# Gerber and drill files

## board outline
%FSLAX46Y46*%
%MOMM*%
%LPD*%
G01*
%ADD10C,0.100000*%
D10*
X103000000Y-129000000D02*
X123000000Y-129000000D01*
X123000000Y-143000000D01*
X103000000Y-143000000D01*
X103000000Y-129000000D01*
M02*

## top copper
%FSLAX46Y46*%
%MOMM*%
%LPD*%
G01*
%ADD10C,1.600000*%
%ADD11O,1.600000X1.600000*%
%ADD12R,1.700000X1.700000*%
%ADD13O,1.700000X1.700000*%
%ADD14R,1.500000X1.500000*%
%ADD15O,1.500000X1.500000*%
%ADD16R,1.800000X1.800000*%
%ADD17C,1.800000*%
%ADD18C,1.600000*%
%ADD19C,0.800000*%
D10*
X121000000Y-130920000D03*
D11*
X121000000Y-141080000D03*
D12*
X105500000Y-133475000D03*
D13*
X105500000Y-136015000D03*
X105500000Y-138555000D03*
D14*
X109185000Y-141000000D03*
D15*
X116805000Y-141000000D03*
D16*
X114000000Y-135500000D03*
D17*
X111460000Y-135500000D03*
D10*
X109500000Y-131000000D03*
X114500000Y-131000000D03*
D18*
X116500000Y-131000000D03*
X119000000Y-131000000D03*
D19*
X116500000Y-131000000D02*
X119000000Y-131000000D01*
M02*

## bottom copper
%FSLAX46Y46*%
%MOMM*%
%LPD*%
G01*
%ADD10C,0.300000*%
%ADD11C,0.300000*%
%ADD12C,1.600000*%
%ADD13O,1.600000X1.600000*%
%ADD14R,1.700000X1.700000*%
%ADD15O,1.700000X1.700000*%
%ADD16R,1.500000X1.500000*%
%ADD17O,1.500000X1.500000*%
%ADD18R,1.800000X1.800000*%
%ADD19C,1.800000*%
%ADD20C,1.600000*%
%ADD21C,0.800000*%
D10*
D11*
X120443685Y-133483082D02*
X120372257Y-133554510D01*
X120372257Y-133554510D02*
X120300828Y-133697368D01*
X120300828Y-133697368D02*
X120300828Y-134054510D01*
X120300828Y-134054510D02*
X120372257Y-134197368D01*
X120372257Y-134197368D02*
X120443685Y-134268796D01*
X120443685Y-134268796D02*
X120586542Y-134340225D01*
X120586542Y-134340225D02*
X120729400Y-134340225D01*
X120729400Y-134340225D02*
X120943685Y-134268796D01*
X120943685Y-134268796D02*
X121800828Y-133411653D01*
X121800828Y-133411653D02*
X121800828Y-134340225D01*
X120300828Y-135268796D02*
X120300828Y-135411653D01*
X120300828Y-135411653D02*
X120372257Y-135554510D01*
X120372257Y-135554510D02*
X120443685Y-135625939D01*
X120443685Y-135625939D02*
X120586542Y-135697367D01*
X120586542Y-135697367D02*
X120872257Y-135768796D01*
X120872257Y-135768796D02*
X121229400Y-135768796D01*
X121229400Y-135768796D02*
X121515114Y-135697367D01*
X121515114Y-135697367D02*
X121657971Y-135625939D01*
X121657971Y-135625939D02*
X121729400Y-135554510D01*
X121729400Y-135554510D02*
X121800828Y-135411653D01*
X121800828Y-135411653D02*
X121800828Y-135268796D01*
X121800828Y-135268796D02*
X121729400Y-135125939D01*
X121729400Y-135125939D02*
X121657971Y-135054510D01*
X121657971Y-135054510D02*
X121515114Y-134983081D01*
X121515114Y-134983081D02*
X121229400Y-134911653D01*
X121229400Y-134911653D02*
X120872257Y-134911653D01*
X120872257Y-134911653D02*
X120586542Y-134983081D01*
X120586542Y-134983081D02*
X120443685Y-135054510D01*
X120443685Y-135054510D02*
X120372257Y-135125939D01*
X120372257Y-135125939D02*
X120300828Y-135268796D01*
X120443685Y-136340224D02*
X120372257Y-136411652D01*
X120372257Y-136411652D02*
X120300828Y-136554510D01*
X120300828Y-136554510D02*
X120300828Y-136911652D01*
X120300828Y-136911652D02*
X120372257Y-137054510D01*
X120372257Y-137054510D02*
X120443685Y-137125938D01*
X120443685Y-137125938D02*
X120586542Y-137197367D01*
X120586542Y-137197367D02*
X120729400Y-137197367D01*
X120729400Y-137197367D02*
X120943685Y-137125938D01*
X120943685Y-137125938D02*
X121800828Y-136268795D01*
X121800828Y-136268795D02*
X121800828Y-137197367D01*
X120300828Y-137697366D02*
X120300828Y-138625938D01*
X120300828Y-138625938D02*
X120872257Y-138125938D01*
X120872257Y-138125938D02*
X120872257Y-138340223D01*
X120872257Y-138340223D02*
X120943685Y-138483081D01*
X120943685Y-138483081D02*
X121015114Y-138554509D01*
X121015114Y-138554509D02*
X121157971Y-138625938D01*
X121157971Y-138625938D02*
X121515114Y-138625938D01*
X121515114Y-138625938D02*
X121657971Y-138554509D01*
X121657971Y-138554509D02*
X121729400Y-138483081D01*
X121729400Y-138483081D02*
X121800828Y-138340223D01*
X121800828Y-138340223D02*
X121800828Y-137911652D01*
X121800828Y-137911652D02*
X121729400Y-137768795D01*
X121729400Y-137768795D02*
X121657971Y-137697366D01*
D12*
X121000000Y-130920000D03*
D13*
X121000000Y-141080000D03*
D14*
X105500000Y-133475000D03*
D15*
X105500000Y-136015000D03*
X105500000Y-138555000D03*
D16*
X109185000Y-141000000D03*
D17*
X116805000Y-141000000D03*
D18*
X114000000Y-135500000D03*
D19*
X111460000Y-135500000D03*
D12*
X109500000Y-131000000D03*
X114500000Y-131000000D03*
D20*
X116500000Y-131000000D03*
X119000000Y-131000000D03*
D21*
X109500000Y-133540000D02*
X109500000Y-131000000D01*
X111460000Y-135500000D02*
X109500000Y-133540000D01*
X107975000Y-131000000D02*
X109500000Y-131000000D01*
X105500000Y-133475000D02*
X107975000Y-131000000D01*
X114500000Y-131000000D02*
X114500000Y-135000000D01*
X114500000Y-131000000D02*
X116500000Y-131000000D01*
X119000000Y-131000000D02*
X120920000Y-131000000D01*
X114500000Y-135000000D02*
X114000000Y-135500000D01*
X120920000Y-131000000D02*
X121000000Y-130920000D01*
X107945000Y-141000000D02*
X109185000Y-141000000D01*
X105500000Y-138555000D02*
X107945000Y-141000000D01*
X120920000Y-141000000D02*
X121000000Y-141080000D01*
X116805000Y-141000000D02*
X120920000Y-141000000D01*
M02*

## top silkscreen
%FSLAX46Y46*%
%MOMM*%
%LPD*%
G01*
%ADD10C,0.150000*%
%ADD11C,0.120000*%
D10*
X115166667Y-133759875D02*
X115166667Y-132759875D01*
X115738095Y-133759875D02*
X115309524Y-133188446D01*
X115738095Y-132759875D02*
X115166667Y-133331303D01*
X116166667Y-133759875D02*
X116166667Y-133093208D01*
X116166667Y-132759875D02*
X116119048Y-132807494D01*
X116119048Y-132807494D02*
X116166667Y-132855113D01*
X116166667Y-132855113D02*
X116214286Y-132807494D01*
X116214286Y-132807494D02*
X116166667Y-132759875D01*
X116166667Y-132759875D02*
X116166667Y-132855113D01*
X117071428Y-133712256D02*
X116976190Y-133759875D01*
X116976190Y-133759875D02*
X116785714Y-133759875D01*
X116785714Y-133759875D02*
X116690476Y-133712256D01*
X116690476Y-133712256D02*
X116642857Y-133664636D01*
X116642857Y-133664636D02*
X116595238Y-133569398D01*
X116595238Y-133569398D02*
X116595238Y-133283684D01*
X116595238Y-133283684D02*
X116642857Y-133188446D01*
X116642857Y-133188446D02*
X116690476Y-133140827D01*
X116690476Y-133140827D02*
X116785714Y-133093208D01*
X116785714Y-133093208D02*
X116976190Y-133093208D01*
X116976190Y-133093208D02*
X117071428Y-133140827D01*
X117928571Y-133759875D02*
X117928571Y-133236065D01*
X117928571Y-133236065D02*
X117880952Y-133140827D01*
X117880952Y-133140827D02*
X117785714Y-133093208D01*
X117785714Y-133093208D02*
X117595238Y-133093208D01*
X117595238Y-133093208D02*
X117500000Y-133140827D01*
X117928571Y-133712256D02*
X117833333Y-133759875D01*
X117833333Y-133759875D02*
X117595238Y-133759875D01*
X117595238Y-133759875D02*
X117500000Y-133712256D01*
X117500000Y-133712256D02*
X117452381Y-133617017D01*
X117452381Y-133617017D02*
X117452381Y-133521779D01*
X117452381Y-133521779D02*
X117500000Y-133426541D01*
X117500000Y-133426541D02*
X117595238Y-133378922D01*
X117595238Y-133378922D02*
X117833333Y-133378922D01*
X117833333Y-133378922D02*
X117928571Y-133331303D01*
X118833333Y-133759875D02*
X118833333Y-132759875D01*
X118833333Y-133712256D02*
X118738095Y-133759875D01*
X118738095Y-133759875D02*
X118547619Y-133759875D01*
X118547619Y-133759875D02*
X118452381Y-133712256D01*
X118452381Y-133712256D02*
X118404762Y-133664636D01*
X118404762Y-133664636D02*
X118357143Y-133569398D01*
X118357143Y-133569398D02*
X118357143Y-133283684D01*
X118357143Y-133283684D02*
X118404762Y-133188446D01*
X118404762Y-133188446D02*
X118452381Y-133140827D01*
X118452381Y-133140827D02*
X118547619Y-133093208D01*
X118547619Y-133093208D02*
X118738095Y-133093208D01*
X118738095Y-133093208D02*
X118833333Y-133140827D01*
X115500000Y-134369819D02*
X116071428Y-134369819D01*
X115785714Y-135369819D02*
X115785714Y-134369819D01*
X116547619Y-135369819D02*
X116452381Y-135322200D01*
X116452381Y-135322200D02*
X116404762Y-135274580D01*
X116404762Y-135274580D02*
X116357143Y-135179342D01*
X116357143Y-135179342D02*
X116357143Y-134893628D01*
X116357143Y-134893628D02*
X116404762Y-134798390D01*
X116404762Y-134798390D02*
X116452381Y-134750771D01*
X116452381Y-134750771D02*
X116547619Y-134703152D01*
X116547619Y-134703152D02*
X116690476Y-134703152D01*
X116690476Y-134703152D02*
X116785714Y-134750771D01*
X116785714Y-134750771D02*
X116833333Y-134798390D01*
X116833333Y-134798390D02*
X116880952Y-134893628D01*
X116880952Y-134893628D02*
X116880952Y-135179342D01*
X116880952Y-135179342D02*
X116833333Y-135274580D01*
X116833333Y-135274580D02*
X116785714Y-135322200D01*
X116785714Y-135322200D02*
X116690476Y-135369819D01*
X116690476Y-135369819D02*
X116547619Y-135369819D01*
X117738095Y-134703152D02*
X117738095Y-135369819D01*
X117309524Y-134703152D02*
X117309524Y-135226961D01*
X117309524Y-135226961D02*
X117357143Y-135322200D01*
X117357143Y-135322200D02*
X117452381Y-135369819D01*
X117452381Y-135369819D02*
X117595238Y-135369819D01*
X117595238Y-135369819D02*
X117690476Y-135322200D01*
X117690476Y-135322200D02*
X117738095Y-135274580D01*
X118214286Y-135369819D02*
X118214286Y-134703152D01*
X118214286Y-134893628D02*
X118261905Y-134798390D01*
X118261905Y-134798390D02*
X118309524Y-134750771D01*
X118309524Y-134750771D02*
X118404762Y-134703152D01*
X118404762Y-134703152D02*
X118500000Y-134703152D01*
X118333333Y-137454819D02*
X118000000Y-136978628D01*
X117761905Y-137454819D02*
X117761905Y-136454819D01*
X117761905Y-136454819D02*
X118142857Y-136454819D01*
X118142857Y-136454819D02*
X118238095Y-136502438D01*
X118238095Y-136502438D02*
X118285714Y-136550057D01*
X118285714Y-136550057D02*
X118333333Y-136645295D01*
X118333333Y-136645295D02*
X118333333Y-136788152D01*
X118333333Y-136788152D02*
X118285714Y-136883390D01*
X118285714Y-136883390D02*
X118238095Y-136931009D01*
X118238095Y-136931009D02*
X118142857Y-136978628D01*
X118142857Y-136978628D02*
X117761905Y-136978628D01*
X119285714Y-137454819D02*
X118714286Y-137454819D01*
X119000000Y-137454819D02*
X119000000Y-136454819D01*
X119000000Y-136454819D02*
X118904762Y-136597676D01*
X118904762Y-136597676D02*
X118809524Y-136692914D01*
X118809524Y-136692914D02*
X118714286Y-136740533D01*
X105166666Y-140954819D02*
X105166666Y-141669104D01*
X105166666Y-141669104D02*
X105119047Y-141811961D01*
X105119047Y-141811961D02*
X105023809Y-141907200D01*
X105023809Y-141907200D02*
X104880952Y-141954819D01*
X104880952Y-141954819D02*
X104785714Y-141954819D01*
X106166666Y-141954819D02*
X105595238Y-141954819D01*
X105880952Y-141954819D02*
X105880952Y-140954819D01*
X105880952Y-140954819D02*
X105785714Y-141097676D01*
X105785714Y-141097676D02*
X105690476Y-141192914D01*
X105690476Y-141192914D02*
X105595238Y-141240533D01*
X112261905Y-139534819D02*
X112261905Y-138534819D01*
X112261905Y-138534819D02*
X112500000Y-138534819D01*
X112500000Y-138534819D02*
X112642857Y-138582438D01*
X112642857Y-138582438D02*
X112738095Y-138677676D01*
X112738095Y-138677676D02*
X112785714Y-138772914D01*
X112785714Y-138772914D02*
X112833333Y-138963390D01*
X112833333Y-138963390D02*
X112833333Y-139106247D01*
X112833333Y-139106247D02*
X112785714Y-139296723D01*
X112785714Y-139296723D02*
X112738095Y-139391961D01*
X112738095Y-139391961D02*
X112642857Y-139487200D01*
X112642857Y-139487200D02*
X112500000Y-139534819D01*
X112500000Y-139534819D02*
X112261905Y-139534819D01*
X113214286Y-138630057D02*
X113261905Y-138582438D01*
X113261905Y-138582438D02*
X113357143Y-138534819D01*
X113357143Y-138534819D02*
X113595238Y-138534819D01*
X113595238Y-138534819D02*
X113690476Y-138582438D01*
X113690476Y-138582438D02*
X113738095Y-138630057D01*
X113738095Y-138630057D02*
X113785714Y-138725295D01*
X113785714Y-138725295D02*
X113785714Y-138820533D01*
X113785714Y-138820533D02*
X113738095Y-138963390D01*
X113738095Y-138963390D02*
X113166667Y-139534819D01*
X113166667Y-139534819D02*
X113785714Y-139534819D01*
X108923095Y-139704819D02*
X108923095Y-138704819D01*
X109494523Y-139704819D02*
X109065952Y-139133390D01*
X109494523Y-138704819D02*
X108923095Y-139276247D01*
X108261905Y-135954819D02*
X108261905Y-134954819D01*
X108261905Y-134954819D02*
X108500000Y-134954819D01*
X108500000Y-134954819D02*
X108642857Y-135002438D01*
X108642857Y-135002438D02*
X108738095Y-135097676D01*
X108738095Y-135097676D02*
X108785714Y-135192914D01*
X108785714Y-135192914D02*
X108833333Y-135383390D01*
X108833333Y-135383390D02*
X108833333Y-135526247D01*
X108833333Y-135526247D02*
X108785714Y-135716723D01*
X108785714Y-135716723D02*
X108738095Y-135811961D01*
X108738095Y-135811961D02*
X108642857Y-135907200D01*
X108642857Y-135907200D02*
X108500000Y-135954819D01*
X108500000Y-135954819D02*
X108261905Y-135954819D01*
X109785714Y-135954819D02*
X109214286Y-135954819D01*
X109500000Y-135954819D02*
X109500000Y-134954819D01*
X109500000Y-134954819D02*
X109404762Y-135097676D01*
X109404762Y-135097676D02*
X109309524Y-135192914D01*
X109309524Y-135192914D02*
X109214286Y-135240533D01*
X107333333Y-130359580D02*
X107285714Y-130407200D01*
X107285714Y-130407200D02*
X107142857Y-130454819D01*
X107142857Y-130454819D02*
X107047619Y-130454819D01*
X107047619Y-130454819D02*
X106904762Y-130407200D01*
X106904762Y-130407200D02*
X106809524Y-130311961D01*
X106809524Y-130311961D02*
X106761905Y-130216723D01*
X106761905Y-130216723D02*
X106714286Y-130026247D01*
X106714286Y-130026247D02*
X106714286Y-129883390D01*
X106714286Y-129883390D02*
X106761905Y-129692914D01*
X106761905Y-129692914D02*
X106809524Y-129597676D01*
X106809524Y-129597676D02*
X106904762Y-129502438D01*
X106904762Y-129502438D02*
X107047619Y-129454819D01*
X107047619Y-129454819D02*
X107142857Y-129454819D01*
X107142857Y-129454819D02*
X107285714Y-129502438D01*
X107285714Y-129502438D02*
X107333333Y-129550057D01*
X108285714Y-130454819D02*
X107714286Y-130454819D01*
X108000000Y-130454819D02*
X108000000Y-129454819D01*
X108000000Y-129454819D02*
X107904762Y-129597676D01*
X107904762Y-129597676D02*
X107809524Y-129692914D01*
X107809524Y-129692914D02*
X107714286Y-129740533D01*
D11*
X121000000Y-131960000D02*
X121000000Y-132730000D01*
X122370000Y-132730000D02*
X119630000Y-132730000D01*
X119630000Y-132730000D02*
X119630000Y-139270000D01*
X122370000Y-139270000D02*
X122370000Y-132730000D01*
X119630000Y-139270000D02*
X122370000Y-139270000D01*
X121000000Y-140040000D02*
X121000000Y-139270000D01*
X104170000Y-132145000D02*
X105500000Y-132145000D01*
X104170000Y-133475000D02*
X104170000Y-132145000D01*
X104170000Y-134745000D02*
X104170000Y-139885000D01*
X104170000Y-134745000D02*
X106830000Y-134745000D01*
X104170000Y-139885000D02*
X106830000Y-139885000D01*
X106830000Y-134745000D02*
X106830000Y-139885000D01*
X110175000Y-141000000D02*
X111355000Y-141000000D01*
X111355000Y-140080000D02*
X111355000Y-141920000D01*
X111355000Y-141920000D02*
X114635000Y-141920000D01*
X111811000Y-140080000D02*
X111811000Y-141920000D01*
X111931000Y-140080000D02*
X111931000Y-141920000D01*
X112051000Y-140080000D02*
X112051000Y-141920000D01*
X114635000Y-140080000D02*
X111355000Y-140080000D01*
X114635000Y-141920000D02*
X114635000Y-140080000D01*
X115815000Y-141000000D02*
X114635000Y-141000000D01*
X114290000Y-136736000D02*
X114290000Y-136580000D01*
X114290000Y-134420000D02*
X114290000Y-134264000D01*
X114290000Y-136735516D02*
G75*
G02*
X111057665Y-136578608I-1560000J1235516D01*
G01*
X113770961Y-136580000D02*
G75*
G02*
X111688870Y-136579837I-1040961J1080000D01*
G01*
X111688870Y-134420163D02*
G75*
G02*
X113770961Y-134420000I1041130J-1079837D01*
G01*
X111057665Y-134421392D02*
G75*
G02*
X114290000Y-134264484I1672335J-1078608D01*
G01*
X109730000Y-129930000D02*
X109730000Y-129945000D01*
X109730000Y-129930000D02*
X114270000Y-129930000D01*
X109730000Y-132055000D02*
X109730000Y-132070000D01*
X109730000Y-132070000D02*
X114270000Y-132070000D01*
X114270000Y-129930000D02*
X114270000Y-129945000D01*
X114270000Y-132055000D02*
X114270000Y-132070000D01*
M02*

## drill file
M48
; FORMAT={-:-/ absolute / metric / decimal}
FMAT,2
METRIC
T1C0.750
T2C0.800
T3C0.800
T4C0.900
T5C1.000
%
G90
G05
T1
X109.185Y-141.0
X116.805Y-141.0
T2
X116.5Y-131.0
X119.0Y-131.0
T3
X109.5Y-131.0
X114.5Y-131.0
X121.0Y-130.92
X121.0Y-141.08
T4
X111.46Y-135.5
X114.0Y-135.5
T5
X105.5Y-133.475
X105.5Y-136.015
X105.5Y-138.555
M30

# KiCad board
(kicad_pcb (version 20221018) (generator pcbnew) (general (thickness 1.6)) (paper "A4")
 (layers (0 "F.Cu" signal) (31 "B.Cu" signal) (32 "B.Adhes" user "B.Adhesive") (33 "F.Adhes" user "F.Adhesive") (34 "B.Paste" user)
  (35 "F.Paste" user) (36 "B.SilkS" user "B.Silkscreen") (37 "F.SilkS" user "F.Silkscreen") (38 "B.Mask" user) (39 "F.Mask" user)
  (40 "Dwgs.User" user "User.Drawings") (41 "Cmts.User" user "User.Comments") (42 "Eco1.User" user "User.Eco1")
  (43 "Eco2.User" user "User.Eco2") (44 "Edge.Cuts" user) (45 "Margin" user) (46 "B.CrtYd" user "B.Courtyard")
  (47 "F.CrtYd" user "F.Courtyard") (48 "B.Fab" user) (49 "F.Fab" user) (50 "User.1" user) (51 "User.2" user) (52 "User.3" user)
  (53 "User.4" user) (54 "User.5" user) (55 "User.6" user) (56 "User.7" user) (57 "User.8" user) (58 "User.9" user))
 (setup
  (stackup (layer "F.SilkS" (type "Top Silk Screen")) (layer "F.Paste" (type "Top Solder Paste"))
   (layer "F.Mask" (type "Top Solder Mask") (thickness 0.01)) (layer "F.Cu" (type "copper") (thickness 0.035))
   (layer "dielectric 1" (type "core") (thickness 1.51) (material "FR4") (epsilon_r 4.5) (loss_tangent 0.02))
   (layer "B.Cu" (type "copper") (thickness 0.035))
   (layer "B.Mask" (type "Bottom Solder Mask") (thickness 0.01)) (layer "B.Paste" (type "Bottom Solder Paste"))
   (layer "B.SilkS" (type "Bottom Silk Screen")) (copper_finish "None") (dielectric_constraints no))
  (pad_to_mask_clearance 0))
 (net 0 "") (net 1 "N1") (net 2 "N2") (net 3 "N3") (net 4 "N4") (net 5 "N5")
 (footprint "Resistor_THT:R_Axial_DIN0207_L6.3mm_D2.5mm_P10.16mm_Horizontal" (layer "F.Cu") (at 121 130.92 -90)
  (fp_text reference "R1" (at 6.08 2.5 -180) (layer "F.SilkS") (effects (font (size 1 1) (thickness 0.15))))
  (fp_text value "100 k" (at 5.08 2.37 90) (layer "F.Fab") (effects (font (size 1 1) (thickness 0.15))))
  (fp_line (start 1.04 0) (end 1.81 0) (stroke (width 0.12) (type solid)) (layer "F.SilkS"))
  (fp_line (start 1.81 -1.37) (end 1.81 1.37) (stroke (width 0.12) (type solid)) (layer "F.SilkS"))
  (fp_line (start 1.81 1.37) (end 8.35 1.37) (stroke (width 0.12) (type solid)) (layer "F.SilkS"))
  (fp_line (start 8.35 -1.37) (end 1.81 -1.37) (stroke (width 0.12) (type solid)) (layer "F.SilkS"))
  (fp_line (start 8.35 1.37) (end 8.35 -1.37) (stroke (width 0.12) (type solid)) (layer "F.SilkS"))
  (fp_line (start 9.12 0) (end 8.35 0) (stroke (width 0.12) (type solid)) (layer "F.SilkS"))
  (pad "1" thru_hole circle (at 0 0 270) (size 1.6 1.6) (drill 0.8) (layers "*.Cu" "*.Mask") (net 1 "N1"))
  (pad "2" thru_hole oval (at 10.16 0 270) (size 1.6 1.6) (drill 0.8) (layers "*.Cu" "*.Mask") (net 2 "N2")))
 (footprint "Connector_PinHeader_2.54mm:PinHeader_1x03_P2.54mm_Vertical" (layer "F.Cu") (at 105.5 133.475)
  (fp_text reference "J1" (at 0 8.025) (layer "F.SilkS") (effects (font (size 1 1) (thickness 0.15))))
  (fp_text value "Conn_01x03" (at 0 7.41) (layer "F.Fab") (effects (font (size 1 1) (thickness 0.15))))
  (fp_line (start -1.33 -1.33) (end 0 -1.33) (stroke (width 0.12) (type solid)) (layer "F.SilkS"))
  (fp_line (start -1.33 0) (end -1.33 -1.33) (stroke (width 0.12) (type solid)) (layer "F.SilkS"))
  (fp_line (start -1.33 1.27) (end -1.33 6.41) (stroke (width 0.12) (type solid)) (layer "F.SilkS"))
  (fp_line (start -1.33 1.27) (end 1.33 1.27) (stroke (width 0.12) (type solid)) (layer "F.SilkS"))
  (fp_line (start -1.33 6.41) (end 1.33 6.41) (stroke (width 0.12) (type solid)) (layer "F.SilkS"))
  (fp_line (start 1.33 1.27) (end 1.33 6.41) (stroke (width 0.12) (type solid)) (layer "F.SilkS"))
  (pad "1" thru_hole rect (at 0 0) (size 1.7 1.7) (drill 1) (layers "*.Cu" "*.Mask") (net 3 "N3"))
  (pad "2" thru_hole oval (at 0 2.54) (size 1.7 1.7) (drill 1) (layers "*.Cu" "*.Mask") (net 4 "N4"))
  (pad "3" thru_hole oval (at 0 5.08) (size 1.7 1.7) (drill 1) (layers "*.Cu" "*.Mask") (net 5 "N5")))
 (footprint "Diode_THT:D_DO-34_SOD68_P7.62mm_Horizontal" (layer "F.Cu") (at 109.185 141)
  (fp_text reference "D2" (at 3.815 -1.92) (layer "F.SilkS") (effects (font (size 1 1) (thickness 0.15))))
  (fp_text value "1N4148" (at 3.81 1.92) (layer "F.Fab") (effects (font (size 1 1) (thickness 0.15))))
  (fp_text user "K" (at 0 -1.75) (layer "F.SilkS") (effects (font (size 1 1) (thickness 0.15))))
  (fp_line (start 0.99 0) (end 2.17 0) (stroke (width 0.12) (type solid)) (layer "F.SilkS"))
  (fp_line (start 2.17 -0.92) (end 2.17 0.92) (stroke (width 0.12) (type solid)) (layer "F.SilkS"))
  (fp_line (start 2.17 0.92) (end 5.45 0.92) (stroke (width 0.12) (type solid)) (layer "F.SilkS"))
  (fp_line (start 2.626 -0.92) (end 2.626 0.92) (stroke (width 0.12) (type solid)) (layer "F.SilkS"))
  (fp_line (start 2.746 -0.92) (end 2.746 0.92) (stroke (width 0.12) (type solid)) (layer "F.SilkS"))
  (fp_line (start 2.866 -0.92) (end 2.866 0.92) (stroke (width 0.12) (type solid)) (layer "F.SilkS"))
  (fp_line (start 5.45 -0.92) (end 2.17 -0.92) (stroke (width 0.12) (type solid)) (layer "F.SilkS"))
  (fp_line (start 5.45 0.92) (end 5.45 -0.92) (stroke (width 0.12) (type solid)) (layer "F.SilkS"))
  (fp_line (start 6.63 0) (end 5.45 0) (stroke (width 0.12) (type solid)) (layer "F.SilkS"))
  (pad "1" thru_hole rect (at 0 0) (size 1.5 1.5) (drill 0.75) (layers "*.Cu" "*.Mask") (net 5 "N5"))
  (pad "2" thru_hole oval (at 7.62 0) (size 1.5 1.5) (drill 0.75) (layers "*.Cu" "*.Mask") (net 2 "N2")))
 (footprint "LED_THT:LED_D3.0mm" (layer "F.Cu") (at 114 135.5 180)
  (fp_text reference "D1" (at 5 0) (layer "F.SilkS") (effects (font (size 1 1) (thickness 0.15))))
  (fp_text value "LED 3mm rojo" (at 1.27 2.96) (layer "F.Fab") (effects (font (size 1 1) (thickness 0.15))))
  (fp_line (start -0.29 -1.236) (end -0.29 -1.08) (stroke (width 0.12) (type solid)) (layer "F.SilkS"))
  (fp_line (start -0.29 1.08) (end -0.29 1.236) (stroke (width 0.12) (type solid)) (layer "F.SilkS"))
  (fp_arc (start -0.29 -1.235516) (mid 1.366487 -1.987659) (end 2.942335 -1.078608) (stroke (width 0.12) (type solid)) (layer "F.SilkS"))
  (fp_arc (start 0.229039 -1.08) (mid 1.270117 -1.5) (end 2.31113 -1.079837) (stroke (width 0.12) (type solid)) (layer "F.SilkS"))
  (fp_arc (start 2.31113 1.079837) (mid 1.270117 1.5) (end 0.229039 1.08) (stroke (width 0.12) (type solid)) (layer "F.SilkS"))
  (fp_arc (start 2.942335 1.078608) (mid 1.366487 1.987659) (end -0.29 1.235516) (stroke (width 0.12) (type solid)) (layer "F.SilkS"))
  (pad "1" thru_hole rect (at 0 0 180) (size 1.8 1.8) (drill 0.9) (layers "*.Cu" "*.Mask") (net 1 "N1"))
  (pad "2" thru_hole circle (at 2.54 0 180) (size 1.8 1.8) (drill 0.9) (layers "*.Cu" "*.Mask") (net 3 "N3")))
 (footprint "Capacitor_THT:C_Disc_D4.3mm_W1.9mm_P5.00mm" (layer "F.Cu") (at 109.5 131)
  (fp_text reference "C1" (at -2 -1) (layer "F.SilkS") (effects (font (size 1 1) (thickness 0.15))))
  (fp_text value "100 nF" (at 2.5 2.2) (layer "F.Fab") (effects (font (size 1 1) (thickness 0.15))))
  (fp_line (start 0.23 -1.07) (end 0.23 -1.055) (stroke (width 0.12) (type solid)) (layer "F.SilkS"))
  (fp_line (start 0.23 -1.07) (end 4.77 -1.07) (stroke (width 0.12) (type solid)) (layer "F.SilkS"))
  (fp_line (start 0.23 1.055) (end 0.23 1.07) (stroke (width 0.12) (type solid)) (layer "F.SilkS"))
  (fp_line (start 0.23 1.07) (end 4.77 1.07) (stroke (width 0.12) (type solid)) (layer "F.SilkS"))
  (fp_line (start 4.77 -1.07) (end 4.77 -1.055) (stroke (width 0.12) (type solid)) (layer "F.SilkS"))
  (fp_line (start 4.77 1.055) (end 4.77 1.07) (stroke (width 0.12) (type solid)) (layer "F.SilkS"))
  (pad "1" thru_hole circle (at 0 0) (size 1.6 1.6) (drill 0.8) (layers "*.Cu" "*.Mask") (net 3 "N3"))
  (pad "2" thru_hole circle (at 5 0) (size 1.6 1.6) (drill 0.8) (layers "*.Cu" "*.Mask") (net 1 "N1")))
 (gr_rect (start 103 129) (end 123 143) (stroke (width 0.1) (type default)) (fill none) (layer "Edge.Cuts"))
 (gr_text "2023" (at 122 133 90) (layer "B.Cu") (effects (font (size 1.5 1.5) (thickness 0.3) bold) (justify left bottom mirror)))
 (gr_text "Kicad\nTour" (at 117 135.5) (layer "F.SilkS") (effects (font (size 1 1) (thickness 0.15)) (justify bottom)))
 (segment (start 109.5 133.54) (end 109.5 131) (width 0.8) (layer "B.Cu") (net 3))
 (segment (start 111.46 135.5) (end 109.5 133.54) (width 0.8) (layer "B.Cu") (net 3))
 (segment (start 107.975 131) (end 109.5 131) (width 0.8) (layer "B.Cu") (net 3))
 (segment (start 105.5 133.475) (end 107.975 131) (width 0.8) (layer "B.Cu") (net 3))
 (segment (start 116.5 131) (end 119 131) (width 0.8) (layer "F.Cu") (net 1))
 (via (at 116.5 131) (size 1.6) (drill 0.8) (layers "F.Cu" "B.Cu") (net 1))
 (via (at 119 131) (size 1.6) (drill 0.8) (layers "F.Cu" "B.Cu") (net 1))
 (segment (start 114.5 131) (end 114.5 135) (width 0.8) (layer "B.Cu") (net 1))
 (segment (start 114.5 131) (end 116.5 131) (width 0.8) (layer "B.Cu") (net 1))
 (segment (start 119 131) (end 120.92 131) (width 0.8) (layer "B.Cu") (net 1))
 (segment (start 114.5 135) (end 114 135.5) (width 0.8) (layer "B.Cu") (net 1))
 (segment (start 120.92 131) (end 121 130.92) (width 0.8) (layer "B.Cu") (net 1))
 (segment (start 107.945 141) (end 109.185 141) (width 0.8) (layer "B.Cu") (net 5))
 (segment (start 105.5 138.555) (end 107.945 141) (width 0.8) (layer "B.Cu") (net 5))
 (segment (start 120.92 141) (end 121 141.08) (width 0.8) (layer "B.Cu") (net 2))
 (segment (start 116.805 141) (end 120.92 141) (width 0.8) (layer "B.Cu") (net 2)))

